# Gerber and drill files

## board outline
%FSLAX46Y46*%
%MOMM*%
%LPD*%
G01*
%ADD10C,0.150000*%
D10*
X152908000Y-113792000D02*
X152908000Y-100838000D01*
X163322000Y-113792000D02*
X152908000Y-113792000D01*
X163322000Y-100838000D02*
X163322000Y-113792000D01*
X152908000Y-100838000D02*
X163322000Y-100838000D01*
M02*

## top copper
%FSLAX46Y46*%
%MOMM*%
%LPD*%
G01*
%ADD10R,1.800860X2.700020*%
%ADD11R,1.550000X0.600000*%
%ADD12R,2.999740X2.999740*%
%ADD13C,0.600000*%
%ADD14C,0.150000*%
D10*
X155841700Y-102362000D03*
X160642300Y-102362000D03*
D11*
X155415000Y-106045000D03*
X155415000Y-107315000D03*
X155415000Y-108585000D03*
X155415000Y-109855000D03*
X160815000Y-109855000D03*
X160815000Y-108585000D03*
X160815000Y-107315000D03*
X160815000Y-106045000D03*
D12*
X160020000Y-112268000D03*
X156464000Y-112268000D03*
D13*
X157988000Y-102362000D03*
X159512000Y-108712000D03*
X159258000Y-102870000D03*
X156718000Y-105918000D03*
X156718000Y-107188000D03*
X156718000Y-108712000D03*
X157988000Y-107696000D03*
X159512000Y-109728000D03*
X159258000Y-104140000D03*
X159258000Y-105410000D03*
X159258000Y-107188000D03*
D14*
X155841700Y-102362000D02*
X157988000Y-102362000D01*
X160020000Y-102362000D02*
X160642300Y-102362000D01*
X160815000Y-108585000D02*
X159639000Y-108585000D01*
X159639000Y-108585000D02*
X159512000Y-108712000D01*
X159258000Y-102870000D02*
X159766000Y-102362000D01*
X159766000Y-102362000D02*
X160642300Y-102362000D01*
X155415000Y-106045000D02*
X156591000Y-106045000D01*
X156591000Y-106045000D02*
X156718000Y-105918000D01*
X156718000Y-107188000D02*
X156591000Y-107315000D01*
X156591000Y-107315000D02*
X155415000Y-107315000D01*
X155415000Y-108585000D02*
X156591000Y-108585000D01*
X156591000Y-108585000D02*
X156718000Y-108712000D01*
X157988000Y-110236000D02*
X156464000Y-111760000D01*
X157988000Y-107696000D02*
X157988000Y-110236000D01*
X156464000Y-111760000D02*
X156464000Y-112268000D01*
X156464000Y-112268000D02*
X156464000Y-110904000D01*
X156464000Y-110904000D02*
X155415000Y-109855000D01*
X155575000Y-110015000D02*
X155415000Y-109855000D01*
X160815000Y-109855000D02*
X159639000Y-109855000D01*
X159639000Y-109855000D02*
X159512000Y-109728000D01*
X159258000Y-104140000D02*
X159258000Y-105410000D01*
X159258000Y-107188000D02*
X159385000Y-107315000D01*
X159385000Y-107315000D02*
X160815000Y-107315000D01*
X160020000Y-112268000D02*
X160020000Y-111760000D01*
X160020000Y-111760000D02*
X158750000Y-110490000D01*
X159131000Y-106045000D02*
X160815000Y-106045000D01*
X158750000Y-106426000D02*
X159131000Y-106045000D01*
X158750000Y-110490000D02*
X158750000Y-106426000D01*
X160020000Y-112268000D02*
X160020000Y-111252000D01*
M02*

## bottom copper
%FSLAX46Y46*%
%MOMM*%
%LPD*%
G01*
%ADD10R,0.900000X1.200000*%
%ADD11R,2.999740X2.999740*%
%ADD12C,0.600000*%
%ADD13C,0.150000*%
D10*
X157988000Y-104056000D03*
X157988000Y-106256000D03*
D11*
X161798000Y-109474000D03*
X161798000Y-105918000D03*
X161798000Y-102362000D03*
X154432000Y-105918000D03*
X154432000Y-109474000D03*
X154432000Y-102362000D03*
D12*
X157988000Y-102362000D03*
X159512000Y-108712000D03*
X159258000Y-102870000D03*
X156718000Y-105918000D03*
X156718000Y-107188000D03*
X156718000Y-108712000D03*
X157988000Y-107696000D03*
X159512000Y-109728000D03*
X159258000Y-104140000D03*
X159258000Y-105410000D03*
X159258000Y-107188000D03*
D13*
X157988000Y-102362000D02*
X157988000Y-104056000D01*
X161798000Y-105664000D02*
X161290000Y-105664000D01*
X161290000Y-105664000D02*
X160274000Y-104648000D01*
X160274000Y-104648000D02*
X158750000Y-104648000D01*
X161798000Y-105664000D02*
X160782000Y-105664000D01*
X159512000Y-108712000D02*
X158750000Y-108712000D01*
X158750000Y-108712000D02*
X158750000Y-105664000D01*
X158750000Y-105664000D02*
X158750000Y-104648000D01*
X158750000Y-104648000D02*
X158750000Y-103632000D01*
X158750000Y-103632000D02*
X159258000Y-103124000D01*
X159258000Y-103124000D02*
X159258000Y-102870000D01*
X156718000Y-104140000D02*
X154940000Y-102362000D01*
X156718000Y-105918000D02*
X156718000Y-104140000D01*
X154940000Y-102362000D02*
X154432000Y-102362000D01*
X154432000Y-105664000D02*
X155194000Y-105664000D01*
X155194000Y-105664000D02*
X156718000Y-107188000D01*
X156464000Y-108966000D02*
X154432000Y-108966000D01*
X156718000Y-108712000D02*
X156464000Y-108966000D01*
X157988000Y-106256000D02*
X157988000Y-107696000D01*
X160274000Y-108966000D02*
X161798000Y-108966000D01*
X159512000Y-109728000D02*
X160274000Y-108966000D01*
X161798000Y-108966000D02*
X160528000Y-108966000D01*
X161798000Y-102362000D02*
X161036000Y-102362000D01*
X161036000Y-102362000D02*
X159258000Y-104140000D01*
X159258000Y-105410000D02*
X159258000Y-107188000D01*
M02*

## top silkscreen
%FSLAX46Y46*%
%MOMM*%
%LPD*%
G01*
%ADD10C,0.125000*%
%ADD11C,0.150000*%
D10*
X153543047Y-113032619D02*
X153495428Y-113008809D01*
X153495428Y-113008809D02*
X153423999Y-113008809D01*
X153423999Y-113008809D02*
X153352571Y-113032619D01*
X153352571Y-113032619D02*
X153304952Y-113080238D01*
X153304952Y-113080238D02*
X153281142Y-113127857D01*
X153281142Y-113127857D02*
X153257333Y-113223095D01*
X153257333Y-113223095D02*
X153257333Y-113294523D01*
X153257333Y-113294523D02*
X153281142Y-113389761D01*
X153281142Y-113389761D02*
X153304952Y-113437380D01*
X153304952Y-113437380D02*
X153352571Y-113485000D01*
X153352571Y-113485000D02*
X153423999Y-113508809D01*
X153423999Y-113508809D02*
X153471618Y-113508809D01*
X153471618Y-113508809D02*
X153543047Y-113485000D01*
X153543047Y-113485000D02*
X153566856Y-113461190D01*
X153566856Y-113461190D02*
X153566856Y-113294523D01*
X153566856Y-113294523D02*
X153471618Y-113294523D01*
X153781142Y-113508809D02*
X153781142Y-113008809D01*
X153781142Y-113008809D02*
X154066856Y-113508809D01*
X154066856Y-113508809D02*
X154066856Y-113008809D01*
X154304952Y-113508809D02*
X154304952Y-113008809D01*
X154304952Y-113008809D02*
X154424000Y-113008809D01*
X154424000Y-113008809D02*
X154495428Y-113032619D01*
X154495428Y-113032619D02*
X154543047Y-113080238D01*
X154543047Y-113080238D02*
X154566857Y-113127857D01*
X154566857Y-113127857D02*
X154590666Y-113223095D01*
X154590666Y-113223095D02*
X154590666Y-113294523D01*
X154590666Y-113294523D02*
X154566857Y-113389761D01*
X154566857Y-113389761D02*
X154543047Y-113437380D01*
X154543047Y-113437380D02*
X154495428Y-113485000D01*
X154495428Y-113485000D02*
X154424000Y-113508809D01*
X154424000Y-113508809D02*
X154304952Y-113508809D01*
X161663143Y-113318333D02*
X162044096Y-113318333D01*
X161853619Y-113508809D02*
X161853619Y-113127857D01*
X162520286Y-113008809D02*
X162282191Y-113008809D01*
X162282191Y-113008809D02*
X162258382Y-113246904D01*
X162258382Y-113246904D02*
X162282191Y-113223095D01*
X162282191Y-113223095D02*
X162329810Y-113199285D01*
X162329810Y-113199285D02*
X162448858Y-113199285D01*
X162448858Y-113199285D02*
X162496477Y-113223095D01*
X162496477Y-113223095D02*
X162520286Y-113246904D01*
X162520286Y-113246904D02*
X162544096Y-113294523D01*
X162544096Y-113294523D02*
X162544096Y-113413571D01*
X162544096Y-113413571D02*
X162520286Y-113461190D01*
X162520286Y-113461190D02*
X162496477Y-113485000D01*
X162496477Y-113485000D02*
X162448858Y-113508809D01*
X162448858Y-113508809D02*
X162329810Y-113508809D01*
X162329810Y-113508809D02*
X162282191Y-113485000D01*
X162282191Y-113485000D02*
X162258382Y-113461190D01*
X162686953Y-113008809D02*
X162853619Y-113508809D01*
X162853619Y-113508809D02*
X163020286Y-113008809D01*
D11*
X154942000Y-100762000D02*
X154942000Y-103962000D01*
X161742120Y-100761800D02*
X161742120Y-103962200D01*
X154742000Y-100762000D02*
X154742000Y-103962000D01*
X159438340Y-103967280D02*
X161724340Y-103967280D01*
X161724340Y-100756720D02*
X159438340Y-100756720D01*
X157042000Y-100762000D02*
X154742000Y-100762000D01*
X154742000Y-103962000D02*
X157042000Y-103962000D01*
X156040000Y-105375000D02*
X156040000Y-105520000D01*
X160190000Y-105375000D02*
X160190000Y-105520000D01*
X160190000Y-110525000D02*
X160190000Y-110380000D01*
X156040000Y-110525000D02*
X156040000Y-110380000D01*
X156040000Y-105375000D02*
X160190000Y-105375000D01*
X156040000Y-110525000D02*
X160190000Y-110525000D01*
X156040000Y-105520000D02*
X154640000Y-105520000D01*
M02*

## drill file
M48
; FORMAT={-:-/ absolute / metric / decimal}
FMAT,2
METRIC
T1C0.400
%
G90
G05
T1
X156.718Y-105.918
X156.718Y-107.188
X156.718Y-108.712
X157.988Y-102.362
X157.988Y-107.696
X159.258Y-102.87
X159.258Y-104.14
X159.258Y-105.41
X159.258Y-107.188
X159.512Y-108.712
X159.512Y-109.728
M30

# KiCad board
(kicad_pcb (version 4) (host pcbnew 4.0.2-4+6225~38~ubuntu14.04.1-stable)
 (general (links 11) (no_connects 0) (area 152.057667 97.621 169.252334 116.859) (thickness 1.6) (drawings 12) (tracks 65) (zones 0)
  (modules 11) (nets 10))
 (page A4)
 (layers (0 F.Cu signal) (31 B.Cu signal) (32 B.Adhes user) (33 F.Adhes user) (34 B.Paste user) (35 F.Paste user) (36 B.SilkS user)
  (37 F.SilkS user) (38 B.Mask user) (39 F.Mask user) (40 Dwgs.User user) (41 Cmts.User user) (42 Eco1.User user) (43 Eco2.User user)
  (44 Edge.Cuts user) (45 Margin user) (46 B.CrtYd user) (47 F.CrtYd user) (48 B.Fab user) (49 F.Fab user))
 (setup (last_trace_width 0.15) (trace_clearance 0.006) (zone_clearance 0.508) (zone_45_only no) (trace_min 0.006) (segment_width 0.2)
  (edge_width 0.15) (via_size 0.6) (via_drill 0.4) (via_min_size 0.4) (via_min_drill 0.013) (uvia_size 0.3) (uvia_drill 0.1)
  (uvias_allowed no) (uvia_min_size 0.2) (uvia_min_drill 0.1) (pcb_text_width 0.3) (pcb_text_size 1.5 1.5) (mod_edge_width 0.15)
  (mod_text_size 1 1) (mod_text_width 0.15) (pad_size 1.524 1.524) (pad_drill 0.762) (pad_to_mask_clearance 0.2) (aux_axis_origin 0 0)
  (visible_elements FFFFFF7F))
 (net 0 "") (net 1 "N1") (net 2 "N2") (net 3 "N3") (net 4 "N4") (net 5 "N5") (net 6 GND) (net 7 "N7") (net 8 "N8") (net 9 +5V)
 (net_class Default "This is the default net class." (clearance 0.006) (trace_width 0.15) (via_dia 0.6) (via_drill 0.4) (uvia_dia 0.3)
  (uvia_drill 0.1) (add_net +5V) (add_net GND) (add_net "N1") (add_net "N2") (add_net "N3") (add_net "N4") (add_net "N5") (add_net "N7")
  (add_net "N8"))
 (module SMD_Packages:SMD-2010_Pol (layer F.Cu) (at 158.242 102.362)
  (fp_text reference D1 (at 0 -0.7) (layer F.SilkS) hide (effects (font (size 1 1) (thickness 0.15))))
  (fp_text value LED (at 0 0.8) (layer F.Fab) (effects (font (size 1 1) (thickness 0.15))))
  (fp_line (start -3.3 -1.6) (end -3.3 1.6) (layer F.SilkS) (width 0.15))
  (fp_line (start 3.50012 -1.6002) (end 3.50012 1.6002) (layer F.SilkS) (width 0.15))
  (fp_line (start -3.5 -1.6) (end -3.5 1.6) (layer F.SilkS) (width 0.15))
  (fp_line (start 1.19634 1.60528) (end 3.48234 1.60528) (layer F.SilkS) (width 0.15))
  (fp_line (start 3.48234 -1.60528) (end 1.19634 -1.60528) (layer F.SilkS) (width 0.15))
  (fp_line (start -1.2 -1.6) (end -3.5 -1.6) (layer F.SilkS) (width 0.15))
  (fp_line (start -3.5 1.6) (end -1.2 1.6) (layer F.SilkS) (width 0.15))
  (pad 1 smd rect (at -2.4003 0) (size 1.80086 2.70002) (layers F.Cu F.Paste F.Mask) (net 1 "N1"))
  (pad 2 smd rect (at 2.4003 0) (size 1.80086 2.70002) (layers F.Cu F.Paste F.Mask) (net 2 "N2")))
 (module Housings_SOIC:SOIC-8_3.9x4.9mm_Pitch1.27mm (layer F.Cu) (at 158.115 107.95)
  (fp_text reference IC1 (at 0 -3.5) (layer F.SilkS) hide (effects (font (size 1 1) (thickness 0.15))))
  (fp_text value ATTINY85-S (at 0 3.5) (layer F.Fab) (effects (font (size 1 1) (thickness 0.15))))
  (fp_line (start -2.075 -2.575) (end -2.075 -2.43) (layer F.SilkS) (width 0.15))
  (fp_line (start 2.075 -2.575) (end 2.075 -2.43) (layer F.SilkS) (width 0.15))
  (fp_line (start 2.075 2.575) (end 2.075 2.43) (layer F.SilkS) (width 0.15))
  (fp_line (start -2.075 2.575) (end -2.075 2.43) (layer F.SilkS) (width 0.15))
  (fp_line (start -2.075 -2.575) (end 2.075 -2.575) (layer F.SilkS) (width 0.15))
  (fp_line (start -2.075 2.575) (end 2.075 2.575) (layer F.SilkS) (width 0.15))
  (fp_line (start -2.075 -2.43) (end -3.475 -2.43) (layer F.SilkS) (width 0.15))
  (pad 1 smd rect (at -2.7 -1.905) (size 1.55 0.6) (layers F.Cu F.Paste F.Mask) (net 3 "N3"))
  (pad 2 smd rect (at -2.7 -0.635) (size 1.55 0.6) (layers F.Cu F.Paste F.Mask) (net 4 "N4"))
  (pad 3 smd rect (at -2.7 0.635) (size 1.55 0.6) (layers F.Cu F.Paste F.Mask) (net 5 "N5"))
  (pad 4 smd rect (at -2.7 1.905) (size 1.55 0.6) (layers F.Cu F.Paste F.Mask) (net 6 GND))
  (pad 5 smd rect (at 2.7 1.905) (size 1.55 0.6) (layers F.Cu F.Paste F.Mask) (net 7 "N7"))
  (pad 6 smd rect (at 2.7 0.635) (size 1.55 0.6) (layers F.Cu F.Paste F.Mask) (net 2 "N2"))
  (pad 7 smd rect (at 2.7 -0.635) (size 1.55 0.6) (layers F.Cu F.Paste F.Mask) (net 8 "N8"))
  (pad 8 smd rect (at 2.7 -1.905) (size 1.55 0.6) (layers F.Cu F.Paste F.Mask) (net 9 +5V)))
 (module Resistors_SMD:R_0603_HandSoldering (layer B.Cu) (at 157.988 105.156 270)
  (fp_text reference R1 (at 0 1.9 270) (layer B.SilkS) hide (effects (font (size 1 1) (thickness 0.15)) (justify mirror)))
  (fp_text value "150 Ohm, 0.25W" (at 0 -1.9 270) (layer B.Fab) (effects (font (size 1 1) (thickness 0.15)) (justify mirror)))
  (pad 1 smd rect (at -1.1 0 270) (size 1.2 0.9) (layers B.Cu B.Paste B.Mask) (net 1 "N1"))
  (pad 2 smd rect (at 1.1 0 270) (size 1.2 0.9) (layers B.Cu B.Paste B.Mask) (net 6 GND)))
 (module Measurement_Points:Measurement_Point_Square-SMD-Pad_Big (layer B.Cu) (at 161.798 109.474)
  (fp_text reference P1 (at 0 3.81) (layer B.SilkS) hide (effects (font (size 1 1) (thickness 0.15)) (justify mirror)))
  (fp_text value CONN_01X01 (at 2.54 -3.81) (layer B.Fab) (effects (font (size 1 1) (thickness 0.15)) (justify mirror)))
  (pad 1 smd rect (at 0 0) (size 2.99974 2.99974) (layers B.Cu B.Mask) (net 7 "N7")))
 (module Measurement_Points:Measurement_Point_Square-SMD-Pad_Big (layer B.Cu) (at 161.798 105.918)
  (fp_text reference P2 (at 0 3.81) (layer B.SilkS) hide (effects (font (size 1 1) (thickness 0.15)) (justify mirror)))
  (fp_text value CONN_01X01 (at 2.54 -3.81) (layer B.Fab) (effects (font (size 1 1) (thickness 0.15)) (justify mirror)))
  (pad 1 smd rect (at 0 0) (size 2.99974 2.99974) (layers B.Cu B.Mask) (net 2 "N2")))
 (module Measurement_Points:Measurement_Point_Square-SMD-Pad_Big (layer B.Cu) (at 161.798 102.362)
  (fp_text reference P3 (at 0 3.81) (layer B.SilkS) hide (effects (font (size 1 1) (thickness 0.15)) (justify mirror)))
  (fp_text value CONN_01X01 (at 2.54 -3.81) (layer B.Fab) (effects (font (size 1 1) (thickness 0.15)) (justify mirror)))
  (pad 1 smd rect (at 0 0) (size 2.99974 2.99974) (layers B.Cu B.Mask) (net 8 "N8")))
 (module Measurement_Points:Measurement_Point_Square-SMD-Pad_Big (layer B.Cu) (at 154.432 105.918)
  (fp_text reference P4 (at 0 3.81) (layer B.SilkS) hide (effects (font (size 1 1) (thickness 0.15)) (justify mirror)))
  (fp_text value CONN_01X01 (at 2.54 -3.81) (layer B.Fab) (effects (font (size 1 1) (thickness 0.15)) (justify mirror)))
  (pad 1 smd rect (at 0 0) (size 2.99974 2.99974) (layers B.Cu B.Mask) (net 4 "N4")))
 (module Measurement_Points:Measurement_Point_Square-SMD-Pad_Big (layer B.Cu) (at 154.432 109.474)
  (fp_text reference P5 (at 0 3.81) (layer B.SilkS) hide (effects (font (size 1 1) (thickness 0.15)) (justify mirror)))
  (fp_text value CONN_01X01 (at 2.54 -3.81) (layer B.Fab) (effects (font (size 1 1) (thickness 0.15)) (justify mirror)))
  (pad 1 smd rect (at 0 0) (size 2.99974 2.99974) (layers B.Cu B.Mask) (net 5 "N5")))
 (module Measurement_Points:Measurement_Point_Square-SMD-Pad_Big (layer B.Cu) (at 154.432 102.362)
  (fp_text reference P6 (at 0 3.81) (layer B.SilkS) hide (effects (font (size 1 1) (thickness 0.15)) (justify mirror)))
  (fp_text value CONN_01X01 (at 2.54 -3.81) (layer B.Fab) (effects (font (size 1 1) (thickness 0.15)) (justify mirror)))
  (pad 1 smd rect (at 0 0) (size 2.99974 2.99974) (layers B.Cu B.Mask) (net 3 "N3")))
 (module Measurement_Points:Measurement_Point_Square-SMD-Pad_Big (layer F.Cu) (at 160.02 112.268)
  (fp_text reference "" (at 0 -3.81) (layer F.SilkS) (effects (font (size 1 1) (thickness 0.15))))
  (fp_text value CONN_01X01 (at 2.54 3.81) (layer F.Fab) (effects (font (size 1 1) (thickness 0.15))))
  (pad 1 smd rect (at 0 0) (size 2.99974 2.99974) (layers F.Cu F.Mask) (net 9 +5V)))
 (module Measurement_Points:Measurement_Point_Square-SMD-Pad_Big (layer F.Cu) (at 156.464 112.268)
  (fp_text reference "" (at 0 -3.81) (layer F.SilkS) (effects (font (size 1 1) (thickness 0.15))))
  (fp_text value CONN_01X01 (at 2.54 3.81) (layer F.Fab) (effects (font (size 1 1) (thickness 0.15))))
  (pad 1 smd rect (at 0 0) (size 2.99974 2.99974) (layers F.Cu F.Mask) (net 6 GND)))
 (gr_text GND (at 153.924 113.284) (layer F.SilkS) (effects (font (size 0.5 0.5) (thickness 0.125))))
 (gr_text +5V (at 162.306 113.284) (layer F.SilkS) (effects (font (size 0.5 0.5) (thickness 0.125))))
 (gr_line (start 152.908 113.792) (end 152.908 100.838) (angle 90) (layer Edge.Cuts) (width 0.15))
 (gr_line (start 163.322 113.792) (end 152.908 113.792) (angle 90) (layer Edge.Cuts) (width 0.15))
 (gr_line (start 163.322 100.838) (end 163.322 113.792) (angle 90) (layer Edge.Cuts) (width 0.15))
 (gr_line (start 152.908 100.838) (end 163.322 100.838) (angle 90) (layer Edge.Cuts) (width 0.15))
 (segment (start 155.8417 102.362) (end 157.988 102.362) (width 0.15) (layer F.Cu) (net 1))
 (segment (start 157.988 102.362) (end 157.988 104.056) (width 0.15) (layer B.Cu) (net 1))
 (via (at 157.988 102.362) (size 0.6) (drill 0.4) (layers F.Cu B.Cu) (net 1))
 (segment (start 161.798 105.664) (end 161.29 105.664) (width 0.15) (layer B.Cu) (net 2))
 (segment (start 161.29 105.664) (end 160.274 104.648) (width 0.15) (layer B.Cu) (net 2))
 (segment (start 160.274 104.648) (end 158.75 104.648) (width 0.15) (layer B.Cu) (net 2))
 (segment (start 161.798 105.664) (end 160.782 105.664) (width 0.15) (layer B.Cu) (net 2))
 (segment (start 160.02 102.362) (end 160.6423 102.362) (width 0.15) (layer F.Cu) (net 2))
 (segment (start 160.815 108.585) (end 159.639 108.585) (width 0.15) (layer F.Cu) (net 2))
 (segment (start 159.639 108.585) (end 159.512 108.712) (width 0.15) (layer F.Cu) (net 2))
 (via (at 159.512 108.712) (size 0.6) (drill 0.4) (layers F.Cu B.Cu) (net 2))
 (segment (start 159.512 108.712) (end 158.75 108.712) (width 0.15) (layer B.Cu) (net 2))
 (segment (start 158.75 108.712) (end 158.75 105.664) (width 0.15) (layer B.Cu) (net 2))
 (segment (start 159.258 102.87) (end 159.766 102.362) (width 0.15) (layer F.Cu) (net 2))
 (segment (start 158.75 105.664) (end 158.75 104.648) (width 0.15) (layer B.Cu) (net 2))
 (segment (start 158.75 104.648) (end 158.75 103.632) (width 0.15) (layer B.Cu) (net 2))
 (segment (start 158.75 103.632) (end 159.258 103.124) (width 0.15) (layer B.Cu) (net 2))
 (segment (start 159.258 103.124) (end 159.258 102.87) (width 0.15) (layer B.Cu) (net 2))
 (via (at 159.258 102.87) (size 0.6) (drill 0.4) (layers F.Cu B.Cu) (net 2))
 (segment (start 159.766 102.362) (end 160.6423 102.362) (width 0.15) (layer F.Cu) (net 2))
 (segment (start 155.415 106.045) (end 156.591 106.045) (width 0.15) (layer F.Cu) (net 3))
 (segment (start 156.718 104.14) (end 154.94 102.362) (width 0.15) (layer B.Cu) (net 3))
 (segment (start 156.718 105.918) (end 156.718 104.14) (width 0.15) (layer B.Cu) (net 3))
 (via (at 156.718 105.918) (size 0.6) (drill 0.4) (layers F.Cu B.Cu) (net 3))
 (segment (start 156.591 106.045) (end 156.718 105.918) (width 0.15) (layer F.Cu) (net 3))
 (segment (start 154.94 102.362) (end 154.432 102.362) (width 0.15) (layer B.Cu) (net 3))
 (segment (start 154.432 105.664) (end 155.194 105.664) (width 0.15) (layer B.Cu) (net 4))
 (segment (start 155.194 105.664) (end 156.718 107.188) (width 0.15) (layer B.Cu) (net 4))
 (via (at 156.718 107.188) (size 0.6) (drill 0.4) (layers F.Cu B.Cu) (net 4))
 (segment (start 156.718 107.188) (end 156.591 107.315) (width 0.15) (layer F.Cu) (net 4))
 (segment (start 156.591 107.315) (end 155.415 107.315) (width 0.15) (layer F.Cu) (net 4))
 (segment (start 155.415 108.585) (end 156.591 108.585) (width 0.15) (layer F.Cu) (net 5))
 (segment (start 156.464 108.966) (end 154.432 108.966) (width 0.15) (layer B.Cu) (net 5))
 (segment (start 156.718 108.712) (end 156.464 108.966) (width 0.15) (layer B.Cu) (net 5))
 (via (at 156.718 108.712) (size 0.6) (drill 0.4) (layers F.Cu B.Cu) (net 5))
 (segment (start 156.591 108.585) (end 156.718 108.712) (width 0.15) (layer F.Cu) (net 5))
 (segment (start 157.988 106.256) (end 157.988 107.696) (width 0.15) (layer B.Cu) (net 6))
 (segment (start 157.988 110.236) (end 156.464 111.76) (width 0.15) (layer F.Cu) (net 6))
 (segment (start 157.988 107.696) (end 157.988 110.236) (width 0.15) (layer F.Cu) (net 6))
 (via (at 157.988 107.696) (size 0.6) (drill 0.4) (layers F.Cu B.Cu) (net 6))
 (segment (start 156.464 111.76) (end 156.464 112.268) (width 0.15) (layer F.Cu) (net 6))
 (segment (start 156.464 112.268) (end 156.464 110.904) (width 0.15) (layer F.Cu) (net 6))
 (segment (start 156.464 110.904) (end 155.415 109.855) (width 0.15) (layer F.Cu) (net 6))
 (segment (start 155.575 110.015) (end 155.415 109.855) (width 0.15) (layer F.Cu) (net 6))
 (segment (start 160.815 109.855) (end 159.639 109.855) (width 0.15) (layer F.Cu) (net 7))
 (segment (start 160.274 108.966) (end 161.798 108.966) (width 0.15) (layer B.Cu) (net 7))
 (segment (start 159.512 109.728) (end 160.274 108.966) (width 0.15) (layer B.Cu) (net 7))
 (via (at 159.512 109.728) (size 0.6) (drill 0.4) (layers F.Cu B.Cu) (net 7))
 (segment (start 159.639 109.855) (end 159.512 109.728) (width 0.15) (layer F.Cu) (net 7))
 (segment (start 161.798 108.966) (end 160.528 108.966) (width 0.15) (layer B.Cu) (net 7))
 (segment (start 161.798 102.362) (end 161.036 102.362) (width 0.15) (layer B.Cu) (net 8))
 (segment (start 161.036 102.362) (end 159.258 104.14) (width 0.15) (layer B.Cu) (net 8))
 (via (at 159.258 104.14) (size 0.6) (drill 0.4) (layers F.Cu B.Cu) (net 8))
 (segment (start 159.258 104.14) (end 159.258 105.41) (width 0.15) (layer F.Cu) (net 8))
 (via (at 159.258 105.41) (size 0.6) (drill 0.4) (layers F.Cu B.Cu) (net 8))
 (segment (start 159.258 105.41) (end 159.258 107.188) (width 0.15) (layer B.Cu) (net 8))
 (via (at 159.258 107.188) (size 0.6) (drill 0.4) (layers F.Cu B.Cu) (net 8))
 (segment (start 159.258 107.188) (end 159.385 107.315) (width 0.15) (layer F.Cu) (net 8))
 (segment (start 159.385 107.315) (end 160.815 107.315) (width 0.15) (layer F.Cu) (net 8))
 (segment (start 160.02 112.268) (end 160.02 111.76) (width 0.15) (layer F.Cu) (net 9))
 (segment (start 160.02 111.76) (end 158.75 110.49) (width 0.15) (layer F.Cu) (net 9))
 (segment (start 159.131 106.045) (end 160.815 106.045) (width 0.15) (layer F.Cu) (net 9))
 (segment (start 158.75 106.426) (end 159.131 106.045) (width 0.15) (layer F.Cu) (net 9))
 (segment (start 158.75 110.49) (end 158.75 106.426) (width 0.15) (layer F.Cu) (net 9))
 (segment (start 160.02 112.268) (end 160.02 111.252) (width 0.15) (layer F.Cu) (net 9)))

